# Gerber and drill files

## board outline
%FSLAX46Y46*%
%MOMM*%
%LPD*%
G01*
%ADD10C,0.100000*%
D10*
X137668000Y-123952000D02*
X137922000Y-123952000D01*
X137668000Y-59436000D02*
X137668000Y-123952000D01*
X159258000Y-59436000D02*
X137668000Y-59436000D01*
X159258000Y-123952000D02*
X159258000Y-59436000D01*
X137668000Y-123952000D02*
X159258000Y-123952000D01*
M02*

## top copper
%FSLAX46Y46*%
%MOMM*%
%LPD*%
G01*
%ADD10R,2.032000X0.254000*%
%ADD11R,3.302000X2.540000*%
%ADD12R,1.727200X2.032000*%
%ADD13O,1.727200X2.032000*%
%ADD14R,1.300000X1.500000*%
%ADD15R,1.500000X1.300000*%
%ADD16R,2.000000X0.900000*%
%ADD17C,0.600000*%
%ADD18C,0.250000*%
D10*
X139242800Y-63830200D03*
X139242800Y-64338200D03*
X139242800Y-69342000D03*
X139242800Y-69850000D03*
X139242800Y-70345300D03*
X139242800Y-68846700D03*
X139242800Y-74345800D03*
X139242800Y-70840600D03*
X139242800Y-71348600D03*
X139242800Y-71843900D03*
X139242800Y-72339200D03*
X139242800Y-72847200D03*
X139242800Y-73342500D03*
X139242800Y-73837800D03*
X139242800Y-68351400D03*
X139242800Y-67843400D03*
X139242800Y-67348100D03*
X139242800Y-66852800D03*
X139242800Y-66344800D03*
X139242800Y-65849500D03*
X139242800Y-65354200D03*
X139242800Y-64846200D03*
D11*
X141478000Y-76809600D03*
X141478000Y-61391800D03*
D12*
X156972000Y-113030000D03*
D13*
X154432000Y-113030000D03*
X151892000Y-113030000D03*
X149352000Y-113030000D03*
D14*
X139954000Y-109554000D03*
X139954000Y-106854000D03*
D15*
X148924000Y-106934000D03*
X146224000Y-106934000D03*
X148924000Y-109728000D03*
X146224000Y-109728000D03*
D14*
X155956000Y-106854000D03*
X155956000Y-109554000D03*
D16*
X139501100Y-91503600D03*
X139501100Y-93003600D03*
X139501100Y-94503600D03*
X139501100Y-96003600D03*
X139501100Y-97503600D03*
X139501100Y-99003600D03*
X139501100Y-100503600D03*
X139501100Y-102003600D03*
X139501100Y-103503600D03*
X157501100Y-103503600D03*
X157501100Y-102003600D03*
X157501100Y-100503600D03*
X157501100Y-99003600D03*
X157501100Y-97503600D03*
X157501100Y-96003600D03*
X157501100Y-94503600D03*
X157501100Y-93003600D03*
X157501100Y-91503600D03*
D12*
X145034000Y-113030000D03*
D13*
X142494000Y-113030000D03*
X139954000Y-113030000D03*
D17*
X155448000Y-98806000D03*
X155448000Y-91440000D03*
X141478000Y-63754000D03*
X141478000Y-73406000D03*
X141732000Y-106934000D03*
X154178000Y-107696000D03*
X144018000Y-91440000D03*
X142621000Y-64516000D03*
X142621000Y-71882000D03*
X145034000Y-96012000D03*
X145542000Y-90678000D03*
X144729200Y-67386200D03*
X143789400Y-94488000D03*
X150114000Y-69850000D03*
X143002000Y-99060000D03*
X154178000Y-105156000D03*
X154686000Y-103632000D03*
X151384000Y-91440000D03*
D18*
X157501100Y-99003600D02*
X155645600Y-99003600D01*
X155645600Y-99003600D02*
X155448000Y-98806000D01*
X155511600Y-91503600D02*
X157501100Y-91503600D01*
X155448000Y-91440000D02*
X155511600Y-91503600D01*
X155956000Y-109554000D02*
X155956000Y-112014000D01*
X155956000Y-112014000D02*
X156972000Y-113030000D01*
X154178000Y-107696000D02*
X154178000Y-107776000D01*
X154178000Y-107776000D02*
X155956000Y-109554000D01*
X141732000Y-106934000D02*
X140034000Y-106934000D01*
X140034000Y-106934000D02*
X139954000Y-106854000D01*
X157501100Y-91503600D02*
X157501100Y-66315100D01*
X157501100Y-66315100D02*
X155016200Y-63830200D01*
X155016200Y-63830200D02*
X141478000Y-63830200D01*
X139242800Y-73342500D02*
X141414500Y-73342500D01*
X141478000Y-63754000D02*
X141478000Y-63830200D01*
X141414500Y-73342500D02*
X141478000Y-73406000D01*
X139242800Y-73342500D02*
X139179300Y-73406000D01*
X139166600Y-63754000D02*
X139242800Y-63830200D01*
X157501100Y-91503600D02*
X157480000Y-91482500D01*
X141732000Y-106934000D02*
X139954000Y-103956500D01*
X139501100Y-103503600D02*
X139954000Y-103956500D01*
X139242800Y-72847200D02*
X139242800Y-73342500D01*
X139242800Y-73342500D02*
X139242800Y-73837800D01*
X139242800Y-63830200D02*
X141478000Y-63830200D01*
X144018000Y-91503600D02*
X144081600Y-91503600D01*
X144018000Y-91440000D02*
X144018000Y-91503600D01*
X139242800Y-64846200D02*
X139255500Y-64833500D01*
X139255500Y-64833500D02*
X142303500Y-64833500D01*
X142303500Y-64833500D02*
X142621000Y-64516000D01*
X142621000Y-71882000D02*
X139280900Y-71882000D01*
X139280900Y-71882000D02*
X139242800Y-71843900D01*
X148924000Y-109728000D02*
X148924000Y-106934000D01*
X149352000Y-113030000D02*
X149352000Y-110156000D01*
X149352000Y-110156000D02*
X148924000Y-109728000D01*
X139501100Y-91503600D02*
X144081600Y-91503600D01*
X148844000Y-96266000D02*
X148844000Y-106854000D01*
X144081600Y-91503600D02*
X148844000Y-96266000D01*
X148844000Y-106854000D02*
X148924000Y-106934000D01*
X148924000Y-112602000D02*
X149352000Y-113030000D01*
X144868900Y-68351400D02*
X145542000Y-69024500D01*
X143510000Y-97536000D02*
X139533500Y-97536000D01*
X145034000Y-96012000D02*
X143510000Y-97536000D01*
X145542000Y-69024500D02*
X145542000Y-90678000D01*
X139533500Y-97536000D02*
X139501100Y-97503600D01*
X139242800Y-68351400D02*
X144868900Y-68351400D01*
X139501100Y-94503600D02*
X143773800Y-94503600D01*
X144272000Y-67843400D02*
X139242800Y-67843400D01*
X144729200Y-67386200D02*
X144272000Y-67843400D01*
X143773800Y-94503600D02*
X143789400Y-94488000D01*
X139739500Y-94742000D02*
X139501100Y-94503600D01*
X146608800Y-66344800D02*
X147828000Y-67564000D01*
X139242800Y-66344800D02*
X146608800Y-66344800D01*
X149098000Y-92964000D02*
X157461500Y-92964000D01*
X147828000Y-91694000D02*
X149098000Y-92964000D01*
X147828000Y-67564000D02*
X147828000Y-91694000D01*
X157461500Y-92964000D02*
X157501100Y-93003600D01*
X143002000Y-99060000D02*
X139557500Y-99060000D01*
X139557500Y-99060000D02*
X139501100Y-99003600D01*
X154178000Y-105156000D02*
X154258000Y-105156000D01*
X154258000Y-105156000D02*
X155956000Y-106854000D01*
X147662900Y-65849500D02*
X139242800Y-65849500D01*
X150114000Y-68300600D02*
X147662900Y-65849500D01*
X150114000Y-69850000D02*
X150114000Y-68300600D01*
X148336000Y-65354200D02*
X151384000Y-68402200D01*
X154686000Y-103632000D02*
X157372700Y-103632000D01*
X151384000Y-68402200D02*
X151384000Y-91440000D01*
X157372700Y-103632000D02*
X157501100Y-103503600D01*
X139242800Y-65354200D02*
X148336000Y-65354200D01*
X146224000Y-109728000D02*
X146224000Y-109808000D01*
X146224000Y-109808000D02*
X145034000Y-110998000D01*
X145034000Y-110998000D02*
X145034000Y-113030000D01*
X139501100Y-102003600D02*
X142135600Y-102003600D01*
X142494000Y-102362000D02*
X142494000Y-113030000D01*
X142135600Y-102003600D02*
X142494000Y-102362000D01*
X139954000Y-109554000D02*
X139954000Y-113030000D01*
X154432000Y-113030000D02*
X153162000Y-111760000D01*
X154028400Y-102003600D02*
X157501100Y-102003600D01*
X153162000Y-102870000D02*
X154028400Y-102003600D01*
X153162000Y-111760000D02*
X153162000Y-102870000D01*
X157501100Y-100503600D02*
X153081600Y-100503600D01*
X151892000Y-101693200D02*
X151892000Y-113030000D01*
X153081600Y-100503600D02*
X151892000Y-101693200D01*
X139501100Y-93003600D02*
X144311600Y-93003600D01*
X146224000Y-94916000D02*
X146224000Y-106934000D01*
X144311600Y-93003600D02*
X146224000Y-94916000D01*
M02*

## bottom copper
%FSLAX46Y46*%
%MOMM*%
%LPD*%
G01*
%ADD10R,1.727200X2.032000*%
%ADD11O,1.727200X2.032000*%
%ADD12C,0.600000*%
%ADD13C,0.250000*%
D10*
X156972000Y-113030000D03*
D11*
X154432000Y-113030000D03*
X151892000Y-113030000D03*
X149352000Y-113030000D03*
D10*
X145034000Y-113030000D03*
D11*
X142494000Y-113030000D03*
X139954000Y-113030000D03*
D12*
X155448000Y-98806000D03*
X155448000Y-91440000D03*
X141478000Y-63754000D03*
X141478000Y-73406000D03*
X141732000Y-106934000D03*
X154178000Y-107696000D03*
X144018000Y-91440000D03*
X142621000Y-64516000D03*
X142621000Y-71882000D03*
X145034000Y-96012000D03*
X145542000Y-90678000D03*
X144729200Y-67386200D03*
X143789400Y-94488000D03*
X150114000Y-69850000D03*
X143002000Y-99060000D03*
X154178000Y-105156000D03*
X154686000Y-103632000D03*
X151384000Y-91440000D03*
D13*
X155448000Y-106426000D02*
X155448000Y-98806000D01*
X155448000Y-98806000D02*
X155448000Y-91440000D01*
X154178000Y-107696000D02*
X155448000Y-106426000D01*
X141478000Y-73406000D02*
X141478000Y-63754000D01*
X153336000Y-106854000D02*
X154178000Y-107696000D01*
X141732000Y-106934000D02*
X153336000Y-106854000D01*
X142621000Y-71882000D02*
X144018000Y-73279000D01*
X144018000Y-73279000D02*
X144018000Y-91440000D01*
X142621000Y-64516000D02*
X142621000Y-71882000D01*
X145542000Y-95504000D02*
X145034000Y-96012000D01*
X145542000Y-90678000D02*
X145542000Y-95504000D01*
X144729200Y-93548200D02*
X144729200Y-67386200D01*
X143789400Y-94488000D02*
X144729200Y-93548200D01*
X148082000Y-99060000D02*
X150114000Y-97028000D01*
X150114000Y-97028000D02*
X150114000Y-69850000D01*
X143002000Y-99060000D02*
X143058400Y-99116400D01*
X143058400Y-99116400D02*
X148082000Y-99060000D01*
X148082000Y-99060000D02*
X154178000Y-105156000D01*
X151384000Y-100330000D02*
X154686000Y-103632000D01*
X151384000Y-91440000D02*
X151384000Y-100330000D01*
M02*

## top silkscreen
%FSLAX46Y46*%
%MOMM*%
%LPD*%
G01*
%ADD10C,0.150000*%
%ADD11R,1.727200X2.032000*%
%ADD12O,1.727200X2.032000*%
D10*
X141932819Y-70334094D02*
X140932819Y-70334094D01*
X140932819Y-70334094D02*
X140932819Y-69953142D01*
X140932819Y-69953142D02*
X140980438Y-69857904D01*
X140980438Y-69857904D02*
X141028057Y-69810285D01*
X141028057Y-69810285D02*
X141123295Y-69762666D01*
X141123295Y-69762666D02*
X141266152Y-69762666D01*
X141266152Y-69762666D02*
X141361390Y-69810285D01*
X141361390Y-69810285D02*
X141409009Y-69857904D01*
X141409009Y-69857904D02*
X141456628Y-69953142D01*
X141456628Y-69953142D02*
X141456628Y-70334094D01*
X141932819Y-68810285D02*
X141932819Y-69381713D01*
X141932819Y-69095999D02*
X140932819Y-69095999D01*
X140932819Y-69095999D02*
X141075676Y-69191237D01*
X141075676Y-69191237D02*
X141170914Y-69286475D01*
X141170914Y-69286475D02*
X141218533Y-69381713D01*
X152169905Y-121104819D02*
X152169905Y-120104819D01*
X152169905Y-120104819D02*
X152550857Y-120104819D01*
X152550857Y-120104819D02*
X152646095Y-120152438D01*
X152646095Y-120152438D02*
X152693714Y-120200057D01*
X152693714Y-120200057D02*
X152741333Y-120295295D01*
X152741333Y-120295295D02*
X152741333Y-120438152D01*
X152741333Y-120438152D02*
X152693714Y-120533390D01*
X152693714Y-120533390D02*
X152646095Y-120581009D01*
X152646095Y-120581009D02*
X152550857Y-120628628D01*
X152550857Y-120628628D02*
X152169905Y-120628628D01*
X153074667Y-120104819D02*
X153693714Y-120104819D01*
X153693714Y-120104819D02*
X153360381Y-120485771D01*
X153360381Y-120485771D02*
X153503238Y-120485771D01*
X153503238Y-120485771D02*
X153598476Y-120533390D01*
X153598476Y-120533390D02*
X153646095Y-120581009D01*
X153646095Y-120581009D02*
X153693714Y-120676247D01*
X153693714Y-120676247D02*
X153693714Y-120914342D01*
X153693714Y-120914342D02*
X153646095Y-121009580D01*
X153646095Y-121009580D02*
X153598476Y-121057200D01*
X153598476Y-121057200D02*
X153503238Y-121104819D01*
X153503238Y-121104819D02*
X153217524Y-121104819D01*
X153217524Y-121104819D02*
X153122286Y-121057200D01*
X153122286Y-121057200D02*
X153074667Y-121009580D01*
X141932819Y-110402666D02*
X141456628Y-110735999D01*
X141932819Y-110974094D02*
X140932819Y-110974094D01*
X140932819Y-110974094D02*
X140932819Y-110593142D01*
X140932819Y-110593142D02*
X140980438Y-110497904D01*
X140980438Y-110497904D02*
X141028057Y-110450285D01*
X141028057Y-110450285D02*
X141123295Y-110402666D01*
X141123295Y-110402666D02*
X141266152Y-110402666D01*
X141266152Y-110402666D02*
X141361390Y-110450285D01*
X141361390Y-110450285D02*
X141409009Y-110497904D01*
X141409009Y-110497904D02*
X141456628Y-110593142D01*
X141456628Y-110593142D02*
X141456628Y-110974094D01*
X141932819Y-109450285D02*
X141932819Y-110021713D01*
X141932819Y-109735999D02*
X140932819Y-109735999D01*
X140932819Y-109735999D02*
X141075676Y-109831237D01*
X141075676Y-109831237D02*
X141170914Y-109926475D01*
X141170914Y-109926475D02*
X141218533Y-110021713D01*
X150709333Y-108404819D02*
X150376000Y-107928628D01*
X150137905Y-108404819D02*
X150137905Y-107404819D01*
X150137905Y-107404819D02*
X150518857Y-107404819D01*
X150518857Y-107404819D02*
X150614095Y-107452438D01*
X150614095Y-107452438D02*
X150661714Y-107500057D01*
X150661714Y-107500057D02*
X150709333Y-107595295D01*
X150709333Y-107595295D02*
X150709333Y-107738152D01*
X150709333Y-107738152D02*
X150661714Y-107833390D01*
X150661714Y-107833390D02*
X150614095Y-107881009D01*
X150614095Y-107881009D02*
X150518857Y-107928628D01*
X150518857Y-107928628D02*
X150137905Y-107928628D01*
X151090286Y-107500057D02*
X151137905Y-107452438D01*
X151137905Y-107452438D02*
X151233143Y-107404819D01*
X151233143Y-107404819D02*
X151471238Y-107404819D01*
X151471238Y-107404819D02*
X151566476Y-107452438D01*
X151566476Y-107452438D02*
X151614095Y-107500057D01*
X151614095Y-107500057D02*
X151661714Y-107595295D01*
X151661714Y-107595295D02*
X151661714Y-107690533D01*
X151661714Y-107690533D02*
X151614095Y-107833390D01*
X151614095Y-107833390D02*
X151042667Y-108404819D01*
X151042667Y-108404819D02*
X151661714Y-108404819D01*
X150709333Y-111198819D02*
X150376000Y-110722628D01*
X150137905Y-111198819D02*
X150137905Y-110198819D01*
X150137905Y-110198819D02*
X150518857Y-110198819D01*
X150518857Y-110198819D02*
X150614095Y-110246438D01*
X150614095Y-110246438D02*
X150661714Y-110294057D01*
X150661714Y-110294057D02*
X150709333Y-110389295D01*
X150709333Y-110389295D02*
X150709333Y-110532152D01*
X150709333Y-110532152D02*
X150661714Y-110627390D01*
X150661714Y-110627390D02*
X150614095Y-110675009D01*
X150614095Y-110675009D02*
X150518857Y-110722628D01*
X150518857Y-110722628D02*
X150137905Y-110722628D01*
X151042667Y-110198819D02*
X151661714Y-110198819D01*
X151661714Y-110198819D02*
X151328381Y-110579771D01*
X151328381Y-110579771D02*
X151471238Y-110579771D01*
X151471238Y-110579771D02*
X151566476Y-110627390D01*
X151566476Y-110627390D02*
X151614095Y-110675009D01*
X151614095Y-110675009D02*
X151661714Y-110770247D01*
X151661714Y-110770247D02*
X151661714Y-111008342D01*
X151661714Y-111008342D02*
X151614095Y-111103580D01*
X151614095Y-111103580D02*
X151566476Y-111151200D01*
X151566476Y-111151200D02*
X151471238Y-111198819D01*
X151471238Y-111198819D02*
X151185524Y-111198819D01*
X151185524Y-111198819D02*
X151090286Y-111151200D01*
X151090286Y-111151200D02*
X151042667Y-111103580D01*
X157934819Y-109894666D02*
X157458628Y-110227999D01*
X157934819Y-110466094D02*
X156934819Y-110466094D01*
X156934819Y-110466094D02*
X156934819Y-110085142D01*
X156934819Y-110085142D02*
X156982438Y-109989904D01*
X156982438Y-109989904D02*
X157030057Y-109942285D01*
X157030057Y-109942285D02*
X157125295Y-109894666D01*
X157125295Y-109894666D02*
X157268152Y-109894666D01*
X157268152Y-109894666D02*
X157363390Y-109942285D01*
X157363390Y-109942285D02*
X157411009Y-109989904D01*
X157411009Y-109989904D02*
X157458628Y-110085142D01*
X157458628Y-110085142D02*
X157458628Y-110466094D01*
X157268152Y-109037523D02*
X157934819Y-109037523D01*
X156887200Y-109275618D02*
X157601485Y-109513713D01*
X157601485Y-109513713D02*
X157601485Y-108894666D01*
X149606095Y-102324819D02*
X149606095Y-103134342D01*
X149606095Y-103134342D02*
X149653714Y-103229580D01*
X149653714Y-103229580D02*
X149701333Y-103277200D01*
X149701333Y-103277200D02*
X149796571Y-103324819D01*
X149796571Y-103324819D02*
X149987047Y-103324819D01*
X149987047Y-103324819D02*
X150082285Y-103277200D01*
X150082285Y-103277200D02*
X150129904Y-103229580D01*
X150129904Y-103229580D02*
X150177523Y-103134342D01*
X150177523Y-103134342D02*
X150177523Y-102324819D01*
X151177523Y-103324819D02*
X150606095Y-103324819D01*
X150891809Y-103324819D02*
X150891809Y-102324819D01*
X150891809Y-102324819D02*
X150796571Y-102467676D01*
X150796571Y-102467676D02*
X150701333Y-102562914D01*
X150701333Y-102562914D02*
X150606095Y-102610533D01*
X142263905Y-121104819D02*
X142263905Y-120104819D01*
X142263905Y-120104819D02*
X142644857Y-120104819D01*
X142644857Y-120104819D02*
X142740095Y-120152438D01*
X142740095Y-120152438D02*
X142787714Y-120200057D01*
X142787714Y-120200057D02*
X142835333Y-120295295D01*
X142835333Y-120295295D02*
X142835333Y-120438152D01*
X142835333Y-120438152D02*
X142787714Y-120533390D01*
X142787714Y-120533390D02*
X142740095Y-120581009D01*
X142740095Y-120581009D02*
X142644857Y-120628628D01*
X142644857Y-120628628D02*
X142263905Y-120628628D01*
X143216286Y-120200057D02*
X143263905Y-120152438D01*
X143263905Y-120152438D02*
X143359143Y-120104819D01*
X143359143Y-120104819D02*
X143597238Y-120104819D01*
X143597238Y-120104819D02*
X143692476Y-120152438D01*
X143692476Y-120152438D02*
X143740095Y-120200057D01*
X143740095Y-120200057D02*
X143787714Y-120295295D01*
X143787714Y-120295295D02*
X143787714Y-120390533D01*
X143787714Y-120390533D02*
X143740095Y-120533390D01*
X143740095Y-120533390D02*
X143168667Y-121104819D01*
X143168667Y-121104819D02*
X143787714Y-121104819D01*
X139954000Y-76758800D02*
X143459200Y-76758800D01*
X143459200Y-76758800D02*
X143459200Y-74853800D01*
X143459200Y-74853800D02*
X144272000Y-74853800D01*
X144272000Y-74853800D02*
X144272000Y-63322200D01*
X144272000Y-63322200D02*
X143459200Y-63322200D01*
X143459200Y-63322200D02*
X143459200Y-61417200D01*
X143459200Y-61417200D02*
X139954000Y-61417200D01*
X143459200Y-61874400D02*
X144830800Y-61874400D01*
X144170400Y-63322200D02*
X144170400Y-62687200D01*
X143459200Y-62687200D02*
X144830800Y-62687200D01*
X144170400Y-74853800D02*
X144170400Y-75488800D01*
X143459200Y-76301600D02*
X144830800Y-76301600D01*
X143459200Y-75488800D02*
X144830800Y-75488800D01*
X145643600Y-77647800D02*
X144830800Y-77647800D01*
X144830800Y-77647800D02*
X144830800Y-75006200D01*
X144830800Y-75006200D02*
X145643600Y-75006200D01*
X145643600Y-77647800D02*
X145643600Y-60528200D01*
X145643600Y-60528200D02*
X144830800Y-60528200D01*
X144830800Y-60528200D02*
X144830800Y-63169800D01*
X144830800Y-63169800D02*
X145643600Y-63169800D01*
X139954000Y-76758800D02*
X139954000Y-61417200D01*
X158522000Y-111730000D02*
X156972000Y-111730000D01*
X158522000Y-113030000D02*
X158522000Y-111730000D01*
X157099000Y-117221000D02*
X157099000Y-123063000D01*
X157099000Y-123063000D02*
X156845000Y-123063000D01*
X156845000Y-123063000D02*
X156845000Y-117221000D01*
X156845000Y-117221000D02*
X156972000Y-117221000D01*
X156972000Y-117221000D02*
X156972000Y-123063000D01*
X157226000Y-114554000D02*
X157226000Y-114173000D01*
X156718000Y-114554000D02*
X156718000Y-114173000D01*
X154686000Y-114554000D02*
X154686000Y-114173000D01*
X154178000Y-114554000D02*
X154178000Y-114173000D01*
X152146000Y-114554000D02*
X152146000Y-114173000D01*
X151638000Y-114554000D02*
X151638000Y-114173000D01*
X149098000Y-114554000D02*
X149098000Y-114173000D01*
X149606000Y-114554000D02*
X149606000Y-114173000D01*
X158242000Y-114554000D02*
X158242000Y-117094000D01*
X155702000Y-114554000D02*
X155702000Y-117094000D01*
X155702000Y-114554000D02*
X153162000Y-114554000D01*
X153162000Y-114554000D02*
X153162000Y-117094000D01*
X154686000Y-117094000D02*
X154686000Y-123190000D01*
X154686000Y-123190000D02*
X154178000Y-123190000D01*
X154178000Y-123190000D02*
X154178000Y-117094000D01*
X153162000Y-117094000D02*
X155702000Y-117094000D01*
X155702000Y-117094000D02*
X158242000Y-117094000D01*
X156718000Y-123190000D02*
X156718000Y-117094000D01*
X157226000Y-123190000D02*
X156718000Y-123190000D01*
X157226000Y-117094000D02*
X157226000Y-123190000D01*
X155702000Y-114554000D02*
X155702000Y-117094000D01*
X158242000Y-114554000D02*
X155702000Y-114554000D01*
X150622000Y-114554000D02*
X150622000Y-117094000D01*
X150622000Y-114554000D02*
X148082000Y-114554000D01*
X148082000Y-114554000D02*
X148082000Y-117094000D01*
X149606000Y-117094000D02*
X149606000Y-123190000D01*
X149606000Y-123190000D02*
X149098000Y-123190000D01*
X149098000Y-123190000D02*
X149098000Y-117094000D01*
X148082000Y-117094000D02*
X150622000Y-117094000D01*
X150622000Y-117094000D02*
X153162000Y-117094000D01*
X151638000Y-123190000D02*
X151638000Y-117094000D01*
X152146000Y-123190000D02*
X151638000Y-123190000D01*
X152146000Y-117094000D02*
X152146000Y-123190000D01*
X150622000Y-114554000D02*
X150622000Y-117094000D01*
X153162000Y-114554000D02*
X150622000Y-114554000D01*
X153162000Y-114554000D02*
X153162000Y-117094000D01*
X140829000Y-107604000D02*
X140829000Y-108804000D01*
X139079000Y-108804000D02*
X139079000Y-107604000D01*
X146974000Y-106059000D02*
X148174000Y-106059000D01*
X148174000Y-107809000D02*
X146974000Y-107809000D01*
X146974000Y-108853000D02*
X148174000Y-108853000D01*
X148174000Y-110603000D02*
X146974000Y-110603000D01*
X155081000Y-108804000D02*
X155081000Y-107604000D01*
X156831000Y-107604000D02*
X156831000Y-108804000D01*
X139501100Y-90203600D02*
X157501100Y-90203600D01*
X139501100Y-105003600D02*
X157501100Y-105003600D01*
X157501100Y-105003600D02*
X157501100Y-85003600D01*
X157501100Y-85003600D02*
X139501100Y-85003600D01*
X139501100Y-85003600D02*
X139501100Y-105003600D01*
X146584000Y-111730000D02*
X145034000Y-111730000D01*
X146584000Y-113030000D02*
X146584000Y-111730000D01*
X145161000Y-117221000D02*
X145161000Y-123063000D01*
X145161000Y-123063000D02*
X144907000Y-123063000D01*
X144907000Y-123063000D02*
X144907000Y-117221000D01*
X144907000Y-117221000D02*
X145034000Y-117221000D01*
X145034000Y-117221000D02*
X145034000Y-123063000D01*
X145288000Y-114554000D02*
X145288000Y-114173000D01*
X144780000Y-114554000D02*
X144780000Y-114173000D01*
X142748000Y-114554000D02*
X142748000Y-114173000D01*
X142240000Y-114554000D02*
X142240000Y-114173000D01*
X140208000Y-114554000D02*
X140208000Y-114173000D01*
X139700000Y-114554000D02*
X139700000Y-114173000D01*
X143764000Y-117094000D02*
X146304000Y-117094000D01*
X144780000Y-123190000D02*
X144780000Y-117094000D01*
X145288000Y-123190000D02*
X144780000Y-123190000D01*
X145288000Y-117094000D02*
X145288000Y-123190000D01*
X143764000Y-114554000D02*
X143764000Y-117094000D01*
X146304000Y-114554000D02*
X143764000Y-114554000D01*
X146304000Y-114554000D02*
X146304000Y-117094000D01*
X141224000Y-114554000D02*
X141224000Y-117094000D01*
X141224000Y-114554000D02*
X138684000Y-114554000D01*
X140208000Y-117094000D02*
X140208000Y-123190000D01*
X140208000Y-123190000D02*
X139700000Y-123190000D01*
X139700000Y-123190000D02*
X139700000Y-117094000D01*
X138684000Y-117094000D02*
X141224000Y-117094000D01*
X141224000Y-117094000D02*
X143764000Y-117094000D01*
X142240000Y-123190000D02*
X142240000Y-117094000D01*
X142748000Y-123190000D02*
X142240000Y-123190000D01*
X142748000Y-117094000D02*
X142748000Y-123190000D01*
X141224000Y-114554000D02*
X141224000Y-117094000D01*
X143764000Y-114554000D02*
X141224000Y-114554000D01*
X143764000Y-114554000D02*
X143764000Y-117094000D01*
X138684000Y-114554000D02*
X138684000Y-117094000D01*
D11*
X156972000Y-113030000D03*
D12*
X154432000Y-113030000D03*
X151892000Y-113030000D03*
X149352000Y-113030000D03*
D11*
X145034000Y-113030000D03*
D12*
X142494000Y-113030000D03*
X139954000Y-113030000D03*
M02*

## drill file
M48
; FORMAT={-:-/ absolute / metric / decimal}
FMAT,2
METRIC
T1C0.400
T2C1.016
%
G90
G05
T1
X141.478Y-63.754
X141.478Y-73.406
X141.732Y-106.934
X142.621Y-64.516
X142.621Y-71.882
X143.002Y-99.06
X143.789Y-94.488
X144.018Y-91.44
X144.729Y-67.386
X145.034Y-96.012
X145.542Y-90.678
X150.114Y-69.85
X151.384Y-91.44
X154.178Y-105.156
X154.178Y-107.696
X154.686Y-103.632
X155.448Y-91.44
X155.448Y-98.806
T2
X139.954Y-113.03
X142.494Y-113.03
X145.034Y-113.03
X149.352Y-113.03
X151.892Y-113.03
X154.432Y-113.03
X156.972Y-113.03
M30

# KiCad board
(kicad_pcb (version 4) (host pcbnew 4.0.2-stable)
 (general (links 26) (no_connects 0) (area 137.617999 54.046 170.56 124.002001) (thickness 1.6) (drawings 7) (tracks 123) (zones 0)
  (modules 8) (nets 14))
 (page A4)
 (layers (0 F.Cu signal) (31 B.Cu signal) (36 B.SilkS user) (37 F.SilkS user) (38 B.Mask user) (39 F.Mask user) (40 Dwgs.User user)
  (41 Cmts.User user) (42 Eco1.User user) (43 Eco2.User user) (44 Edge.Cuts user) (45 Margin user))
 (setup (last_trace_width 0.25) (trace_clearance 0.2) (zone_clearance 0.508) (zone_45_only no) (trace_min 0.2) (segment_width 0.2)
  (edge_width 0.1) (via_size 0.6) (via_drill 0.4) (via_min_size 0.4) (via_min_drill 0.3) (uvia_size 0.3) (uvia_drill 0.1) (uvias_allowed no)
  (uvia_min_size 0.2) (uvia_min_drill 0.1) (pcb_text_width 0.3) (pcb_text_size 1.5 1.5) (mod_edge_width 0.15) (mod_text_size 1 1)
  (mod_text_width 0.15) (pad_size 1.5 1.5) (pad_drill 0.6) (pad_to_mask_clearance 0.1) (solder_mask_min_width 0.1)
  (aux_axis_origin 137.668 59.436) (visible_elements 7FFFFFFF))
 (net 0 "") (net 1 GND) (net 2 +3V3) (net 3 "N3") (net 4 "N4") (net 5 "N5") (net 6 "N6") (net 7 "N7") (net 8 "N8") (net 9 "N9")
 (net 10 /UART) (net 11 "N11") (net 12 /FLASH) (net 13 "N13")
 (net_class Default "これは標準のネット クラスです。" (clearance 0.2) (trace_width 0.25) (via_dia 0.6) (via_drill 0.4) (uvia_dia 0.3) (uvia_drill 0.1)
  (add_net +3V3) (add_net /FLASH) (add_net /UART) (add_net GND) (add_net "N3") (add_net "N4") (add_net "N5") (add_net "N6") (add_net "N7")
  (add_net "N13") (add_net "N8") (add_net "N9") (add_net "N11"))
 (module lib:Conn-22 (layer F.Cu) (at 142.494 69.088 90)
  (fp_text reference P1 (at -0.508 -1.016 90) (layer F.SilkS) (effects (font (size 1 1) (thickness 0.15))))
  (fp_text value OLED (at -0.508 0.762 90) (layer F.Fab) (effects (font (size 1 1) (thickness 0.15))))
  (fp_line (start -7.6708 -2.54) (end -7.6708 0.9652) (layer F.SilkS) (width 0.15))
  (fp_line (start -7.6708 0.9652) (end -5.7658 0.9652) (layer F.SilkS) (width 0.15))
  (fp_line (start -5.7658 0.9652) (end -5.7658 1.778) (layer F.SilkS) (width 0.15))
  (fp_line (start -5.7658 1.778) (end 5.7658 1.778) (layer F.SilkS) (width 0.15))
  (fp_line (start 5.7658 1.778) (end 5.7658 0.9652) (layer F.SilkS) (width 0.15))
  (fp_line (start 5.7658 0.9652) (end 7.6708 0.9652) (layer F.SilkS) (width 0.15))
  (fp_line (start 7.6708 0.9652) (end 7.6708 -2.54) (layer F.SilkS) (width 0.15))
  (fp_line (start 7.2136 0.9652) (end 7.2136 2.3368) (layer F.SilkS) (width 0.15))
  (fp_line (start 5.7658 1.6764) (end 6.4008 1.6764) (layer F.SilkS) (width 0.15))
  (fp_line (start 6.4008 0.9652) (end 6.4008 2.3368) (layer F.SilkS) (width 0.15))
  (fp_line (start -5.7658 1.6764) (end -6.4008 1.6764) (layer F.SilkS) (width 0.15))
  (fp_line (start -7.2136 0.9652) (end -7.2136 2.3368) (layer F.SilkS) (width 0.15))
  (fp_line (start -6.4008 0.9652) (end -6.4008 2.3368) (layer F.SilkS) (width 0.15))
  (fp_line (start -8.5598 3.1496) (end -8.5598 2.3368) (layer F.SilkS) (width 0.15))
  (fp_line (start -8.5598 2.3368) (end -5.9182 2.3368) (layer F.SilkS) (width 0.15))
  (fp_line (start -5.9182 2.3368) (end -5.9182 3.1496) (layer F.SilkS) (width 0.15))
  (fp_line (start -8.5598 3.1496) (end 8.5598 3.1496) (layer F.SilkS) (width 0.15))
  (fp_line (start 8.5598 3.1496) (end 8.5598 2.3368) (layer F.SilkS) (width 0.15))
  (fp_line (start 8.5598 2.3368) (end 5.9182 2.3368) (layer F.SilkS) (width 0.15))
  (fp_line (start 5.9182 2.3368) (end 5.9182 3.1496) (layer F.SilkS) (width 0.15))
  (fp_line (start -7.6708 -2.54) (end 7.6708 -2.54) (layer F.SilkS) (width 0.15))
  (pad 22 smd rect (at 5.2578 -3.2512 90) (size 0.254 2.032) (layers F.Cu F.Mask) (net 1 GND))
  (pad 21 smd rect (at 4.7498 -3.2512 90) (size 0.254 2.032) (layers F.Cu F.Mask))
  (pad 11 smd rect (at -0.254 -3.2512 90) (size 0.254 2.032) (layers F.Cu F.Mask))
  (pad 10 smd rect (at -0.762 -3.2512 90) (size 0.254 2.032) (layers F.Cu F.Mask))
  (pad 9 smd rect (at -1.2573 -3.2512 90) (size 0.254 2.032) (layers F.Cu F.Mask))
  (pad 12 smd rect (at 0.2413 -3.2512 90) (size 0.254 2.032) (layers F.Cu F.Mask))
  (pad 1 smd rect (at -5.2578 -3.2512 90) (size 0.254 2.032) (layers F.Cu F.Mask))
  (pad 8 smd rect (at -1.7526 -3.2512 90) (size 0.254 2.032) (layers F.Cu F.Mask))
  (pad 7 smd rect (at -2.2606 -3.2512 90) (size 0.254 2.032) (layers F.Cu F.Mask))
  (pad 6 smd rect (at -2.7559 -3.2512 90) (size 0.254 2.032) (layers F.Cu F.Mask) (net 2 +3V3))
  (pad 5 smd rect (at -3.2512 -3.2512 90) (size 0.254 2.032) (layers F.Cu F.Mask))
  (pad 4 smd rect (at -3.7592 -3.2512 90) (size 0.254 2.032) (layers F.Cu F.Mask) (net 1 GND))
  (pad 3 smd rect (at -4.2545 -3.2512 90) (size 0.254 2.032) (layers F.Cu F.Mask) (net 1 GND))
  (pad 2 smd rect (at -4.7498 -3.2512 90) (size 0.254 2.032) (layers F.Cu F.Mask) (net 1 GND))
  (pad 13 smd rect (at 0.7366 -3.2512 90) (size 0.254 2.032) (layers F.Cu F.Mask) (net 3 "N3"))
  (pad 14 smd rect (at 1.2446 -3.2512 90) (size 0.254 2.032) (layers F.Cu F.Mask) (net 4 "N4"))
  (pad 15 smd rect (at 1.7399 -3.2512 90) (size 0.254 2.032) (layers F.Cu F.Mask))
  (pad 16 smd rect (at 2.2352 -3.2512 90) (size 0.254 2.032) (layers F.Cu F.Mask))
  (pad 17 smd rect (at 2.7432 -3.2512 90) (size 0.254 2.032) (layers F.Cu F.Mask) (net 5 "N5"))
  (pad 18 smd rect (at 3.2385 -3.2512 90) (size 0.254 2.032) (layers F.Cu F.Mask) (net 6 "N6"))
  (pad 19 smd rect (at 3.7338 -3.2512 90) (size 0.254 2.032) (layers F.Cu F.Mask) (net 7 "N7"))
  (pad 20 smd rect (at 4.2418 -3.2512 90) (size 0.254 2.032) (layers F.Cu F.Mask) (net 2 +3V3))
  (pad "" smd rect (at -7.7216 -1.016 90) (size 2.54 3.302) (layers F.Cu F.Mask))
  (pad "" smd rect (at 7.6962 -1.016 90) (size 2.54 3.302) (layers F.Cu F.Mask)))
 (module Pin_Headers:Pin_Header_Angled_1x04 (layer F.Cu) (at 156.972 113.03 270)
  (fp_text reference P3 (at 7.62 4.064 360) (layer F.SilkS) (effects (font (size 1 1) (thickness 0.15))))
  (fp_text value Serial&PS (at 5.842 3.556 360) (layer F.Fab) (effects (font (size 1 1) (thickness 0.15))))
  (fp_line (start -1.3 -1.55) (end -1.3 0) (layer F.SilkS) (width 0.15))
  (fp_line (start 0 -1.55) (end -1.3 -1.55) (layer F.SilkS) (width 0.15))
  (fp_line (start 4.191 -0.127) (end 10.033 -0.127) (layer F.SilkS) (width 0.15))
  (fp_line (start 10.033 -0.127) (end 10.033 0.127) (layer F.SilkS) (width 0.15))
  (fp_line (start 10.033 0.127) (end 4.191 0.127) (layer F.SilkS) (width 0.15))
  (fp_line (start 4.191 0.127) (end 4.191 0) (layer F.SilkS) (width 0.15))
  (fp_line (start 4.191 0) (end 10.033 0) (layer F.SilkS) (width 0.15))
  (fp_line (start 1.524 -0.254) (end 1.143 -0.254) (layer F.SilkS) (width 0.15))
  (fp_line (start 1.524 0.254) (end 1.143 0.254) (layer F.SilkS) (width 0.15))
  (fp_line (start 1.524 2.286) (end 1.143 2.286) (layer F.SilkS) (width 0.15))
  (fp_line (start 1.524 2.794) (end 1.143 2.794) (layer F.SilkS) (width 0.15))
  (fp_line (start 1.524 4.826) (end 1.143 4.826) (layer F.SilkS) (width 0.15))
  (fp_line (start 1.524 5.334) (end 1.143 5.334) (layer F.SilkS) (width 0.15))
  (fp_line (start 1.524 7.874) (end 1.143 7.874) (layer F.SilkS) (width 0.15))
  (fp_line (start 1.524 7.366) (end 1.143 7.366) (layer F.SilkS) (width 0.15))
  (fp_line (start 1.524 -1.27) (end 4.064 -1.27) (layer F.SilkS) (width 0.15))
  (fp_line (start 1.524 1.27) (end 4.064 1.27) (layer F.SilkS) (width 0.15))
  (fp_line (start 1.524 1.27) (end 1.524 3.81) (layer F.SilkS) (width 0.15))
  (fp_line (start 1.524 3.81) (end 4.064 3.81) (layer F.SilkS) (width 0.15))
  (fp_line (start 4.064 2.286) (end 10.16 2.286) (layer F.SilkS) (width 0.15))
  (fp_line (start 10.16 2.286) (end 10.16 2.794) (layer F.SilkS) (width 0.15))
  (fp_line (start 10.16 2.794) (end 4.064 2.794) (layer F.SilkS) (width 0.15))
  (fp_line (start 4.064 3.81) (end 4.064 1.27) (layer F.SilkS) (width 0.15))
  (fp_line (start 4.064 1.27) (end 4.064 -1.27) (layer F.SilkS) (width 0.15))
  (fp_line (start 10.16 0.254) (end 4.064 0.254) (layer F.SilkS) (width 0.15))
  (fp_line (start 10.16 -0.254) (end 10.16 0.254) (layer F.SilkS) (width 0.15))
  (fp_line (start 4.064 -0.254) (end 10.16 -0.254) (layer F.SilkS) (width 0.15))
  (fp_line (start 1.524 1.27) (end 4.064 1.27) (layer F.SilkS) (width 0.15))
  (fp_line (start 1.524 -1.27) (end 1.524 1.27) (layer F.SilkS) (width 0.15))
  (fp_line (start 1.524 6.35) (end 4.064 6.35) (layer F.SilkS) (width 0.15))
  (fp_line (start 1.524 6.35) (end 1.524 8.89) (layer F.SilkS) (width 0.15))
  (fp_line (start 1.524 8.89) (end 4.064 8.89) (layer F.SilkS) (width 0.15))
  (fp_line (start 4.064 7.366) (end 10.16 7.366) (layer F.SilkS) (width 0.15))
  (fp_line (start 10.16 7.366) (end 10.16 7.874) (layer F.SilkS) (width 0.15))
  (fp_line (start 10.16 7.874) (end 4.064 7.874) (layer F.SilkS) (width 0.15))
  (fp_line (start 4.064 8.89) (end 4.064 6.35) (layer F.SilkS) (width 0.15))
  (fp_line (start 4.064 6.35) (end 4.064 3.81) (layer F.SilkS) (width 0.15))
  (fp_line (start 10.16 5.334) (end 4.064 5.334) (layer F.SilkS) (width 0.15))
  (fp_line (start 10.16 4.826) (end 10.16 5.334) (layer F.SilkS) (width 0.15))
  (fp_line (start 4.064 4.826) (end 10.16 4.826) (layer F.SilkS) (width 0.15))
  (fp_line (start 1.524 6.35) (end 4.064 6.35) (layer F.SilkS) (width 0.15))
  (fp_line (start 1.524 3.81) (end 1.524 6.35) (layer F.SilkS) (width 0.15))
  (fp_line (start 1.524 3.81) (end 4.064 3.81) (layer F.SilkS) (width 0.15))
  (pad 1 thru_hole rect (at 0 0 270) (size 2.032 1.7272) (drill 1.016) (layers *.Cu *.Mask F.SilkS) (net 1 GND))
  (pad 2 thru_hole oval (at 0 2.54 270) (size 2.032 1.7272) (drill 1.016) (layers *.Cu *.Mask F.SilkS) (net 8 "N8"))
  (pad 3 thru_hole oval (at 0 5.08 270) (size 2.032 1.7272) (drill 1.016) (layers *.Cu *.Mask F.SilkS) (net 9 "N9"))
  (pad 4 thru_hole oval (at 0 7.62 270) (size 2.032 1.7272) (drill 1.016) (layers *.Cu *.Mask F.SilkS) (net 2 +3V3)))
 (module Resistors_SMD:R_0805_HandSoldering (layer F.Cu) (at 139.954 108.204 90)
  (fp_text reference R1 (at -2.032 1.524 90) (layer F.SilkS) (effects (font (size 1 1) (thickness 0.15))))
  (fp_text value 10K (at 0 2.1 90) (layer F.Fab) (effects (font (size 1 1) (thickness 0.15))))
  (fp_line (start 0.6 0.875) (end -0.6 0.875) (layer F.SilkS) (width 0.15))
  (fp_line (start -0.6 -0.875) (end 0.6 -0.875) (layer F.SilkS) (width 0.15))
  (pad 1 smd rect (at -1.35 0 90) (size 1.5 1.3) (layers F.Cu F.Mask) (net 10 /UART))
  (pad 2 smd rect (at 1.35 0 90) (size 1.5 1.3) (layers F.Cu F.Mask) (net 1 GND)))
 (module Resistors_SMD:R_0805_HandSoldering (layer F.Cu) (at 147.574 106.934 180)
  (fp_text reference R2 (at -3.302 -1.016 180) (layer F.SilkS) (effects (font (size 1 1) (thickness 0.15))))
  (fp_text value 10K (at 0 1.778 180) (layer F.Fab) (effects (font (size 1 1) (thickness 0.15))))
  (fp_line (start 0.6 0.875) (end -0.6 0.875) (layer F.SilkS) (width 0.15))
  (fp_line (start -0.6 -0.875) (end 0.6 -0.875) (layer F.SilkS) (width 0.15))
  (pad 1 smd rect (at -1.35 0 180) (size 1.5 1.3) (layers F.Cu F.Mask) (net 2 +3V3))
  (pad 2 smd rect (at 1.35 0 180) (size 1.5 1.3) (layers F.Cu F.Mask) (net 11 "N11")))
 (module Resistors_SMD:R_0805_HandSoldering (layer F.Cu) (at 147.574 109.728 180)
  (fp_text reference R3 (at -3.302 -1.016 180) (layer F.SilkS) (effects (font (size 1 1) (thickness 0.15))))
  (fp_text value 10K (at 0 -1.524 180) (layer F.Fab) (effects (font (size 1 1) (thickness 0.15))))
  (fp_line (start 0.6 0.875) (end -0.6 0.875) (layer F.SilkS) (width 0.15))
  (fp_line (start -0.6 -0.875) (end 0.6 -0.875) (layer F.SilkS) (width 0.15))
  (pad 1 smd rect (at -1.35 0 180) (size 1.5 1.3) (layers F.Cu F.Mask) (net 2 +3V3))
  (pad 2 smd rect (at 1.35 0 180) (size 1.5 1.3) (layers F.Cu F.Mask) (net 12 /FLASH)))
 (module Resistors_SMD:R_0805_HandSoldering (layer F.Cu) (at 155.956 108.204 270)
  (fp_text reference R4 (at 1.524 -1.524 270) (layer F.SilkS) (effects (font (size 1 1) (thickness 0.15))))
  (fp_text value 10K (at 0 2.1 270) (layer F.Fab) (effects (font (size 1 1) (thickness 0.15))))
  (fp_line (start 0.6 0.875) (end -0.6 0.875) (layer F.SilkS) (width 0.15))
  (fp_line (start -0.6 -0.875) (end 0.6 -0.875) (layer F.SilkS) (width 0.15))
  (pad 1 smd rect (at -1.35 0 270) (size 1.5 1.3) (layers F.Cu F.Mask) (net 6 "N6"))
  (pad 2 smd rect (at 1.35 0 270) (size 1.5 1.3) (layers F.Cu F.Mask) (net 1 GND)))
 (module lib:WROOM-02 (layer F.Cu) (at 148.5011 105.0036)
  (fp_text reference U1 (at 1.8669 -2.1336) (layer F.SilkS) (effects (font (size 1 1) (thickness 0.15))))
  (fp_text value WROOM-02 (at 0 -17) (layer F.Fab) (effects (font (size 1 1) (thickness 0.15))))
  (fp_line (start -9 -14.8) (end 9 -14.8) (layer F.SilkS) (width 0.15))
  (fp_line (start -9 0) (end 9 0) (layer F.SilkS) (width 0.15))
  (fp_line (start 9 0) (end 9 -20) (layer F.SilkS) (width 0.15))
  (fp_line (start 9 -20) (end -9 -20) (layer F.SilkS) (width 0.15))
  (fp_line (start -9 -20) (end -9 0) (layer F.SilkS) (width 0.15))
  (pad 1 smd rect (at -9 -13.5) (size 2 0.9) (layers F.Cu F.Mask) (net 2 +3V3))
  (pad 2 smd rect (at -9 -12) (size 2 0.9) (layers F.Cu F.Mask) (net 11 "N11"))
  (pad 3 smd rect (at -9 -10.5) (size 2 0.9) (layers F.Cu F.Mask) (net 4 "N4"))
  (pad 4 smd rect (at -9 -9) (size 2 0.9) (layers F.Cu F.Mask))
  (pad 5 smd rect (at -9 -7.5) (size 2 0.9) (layers F.Cu F.Mask) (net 3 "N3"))
  (pad 6 smd rect (at -9 -6) (size 2 0.9) (layers F.Cu F.Mask) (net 6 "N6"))
  (pad 7 smd rect (at -9 -4.5) (size 2 0.9) (layers F.Cu F.Mask))
  (pad 8 smd rect (at -9 -3) (size 2 0.9) (layers F.Cu F.Mask) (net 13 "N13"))
  (pad 9 smd rect (at -9 -1.5) (size 2 0.9) (layers F.Cu F.Mask) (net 1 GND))
  (pad 10 smd rect (at 9 -1.5) (size 2 0.9) (layers F.Cu F.Mask) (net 7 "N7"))
  (pad 11 smd rect (at 9 -3) (size 2 0.9) (layers F.Cu F.Mask) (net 8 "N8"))
  (pad 12 smd rect (at 9 -4.5) (size 2 0.9) (layers F.Cu F.Mask) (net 9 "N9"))
  (pad 13 smd rect (at 9 -6) (size 2 0.9) (layers F.Cu F.Mask) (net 1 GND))
  (pad 14 smd rect (at 9 -7.5) (size 2 0.9) (layers F.Cu F.Mask))
  (pad 15 smd rect (at 9 -9) (size 2 0.9) (layers F.Cu F.Mask))
  (pad 16 smd rect (at 9 -10.5) (size 2 0.9) (layers F.Cu F.Mask))
  (pad 17 smd rect (at 9 -12) (size 2 0.9) (layers F.Cu F.Mask) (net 5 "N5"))
  (pad 18 smd rect (at 9 -13.5) (size 2 0.9) (layers F.Cu F.Mask) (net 1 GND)))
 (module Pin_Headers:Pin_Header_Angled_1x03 (layer F.Cu) (at 145.034 113.03 270)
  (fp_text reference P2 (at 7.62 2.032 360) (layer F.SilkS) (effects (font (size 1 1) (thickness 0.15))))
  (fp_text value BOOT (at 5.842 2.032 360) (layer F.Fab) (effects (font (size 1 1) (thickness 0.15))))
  (fp_line (start -1.3 -1.55) (end -1.3 0) (layer F.SilkS) (width 0.15))
  (fp_line (start 0 -1.55) (end -1.3 -1.55) (layer F.SilkS) (width 0.15))
  (fp_line (start 4.191 -0.127) (end 10.033 -0.127) (layer F.SilkS) (width 0.15))
  (fp_line (start 10.033 -0.127) (end 10.033 0.127) (layer F.SilkS) (width 0.15))
  (fp_line (start 10.033 0.127) (end 4.191 0.127) (layer F.SilkS) (width 0.15))
  (fp_line (start 4.191 0.127) (end 4.191 0) (layer F.SilkS) (width 0.15))
  (fp_line (start 4.191 0) (end 10.033 0) (layer F.SilkS) (width 0.15))
  (fp_line (start 1.524 -0.254) (end 1.143 -0.254) (layer F.SilkS) (width 0.15))
  (fp_line (start 1.524 0.254) (end 1.143 0.254) (layer F.SilkS) (width 0.15))
  (fp_line (start 1.524 2.286) (end 1.143 2.286) (layer F.SilkS) (width 0.15))
  (fp_line (start 1.524 2.794) (end 1.143 2.794) (layer F.SilkS) (width 0.15))
  (fp_line (start 1.524 4.826) (end 1.143 4.826) (layer F.SilkS) (width 0.15))
  (fp_line (start 1.524 5.334) (end 1.143 5.334) (layer F.SilkS) (width 0.15))
  (fp_line (start 4.064 1.27) (end 4.064 -1.27) (layer F.SilkS) (width 0.15))
  (fp_line (start 10.16 0.254) (end 4.064 0.254) (layer F.SilkS) (width 0.15))
  (fp_line (start 10.16 -0.254) (end 10.16 0.254) (layer F.SilkS) (width 0.15))
  (fp_line (start 4.064 -0.254) (end 10.16 -0.254) (layer F.SilkS) (width 0.15))
  (fp_line (start 1.524 1.27) (end 4.064 1.27) (layer F.SilkS) (width 0.15))
  (fp_line (start 1.524 -1.27) (end 1.524 1.27) (layer F.SilkS) (width 0.15))
  (fp_line (start 1.524 -1.27) (end 4.064 -1.27) (layer F.SilkS) (width 0.15))
  (fp_line (start 1.524 3.81) (end 4.064 3.81) (layer F.SilkS) (width 0.15))
  (fp_line (start 1.524 3.81) (end 1.524 6.35) (layer F.SilkS) (width 0.15))
  (fp_line (start 4.064 4.826) (end 10.16 4.826) (layer F.SilkS) (width 0.15))
  (fp_line (start 10.16 4.826) (end 10.16 5.334) (layer F.SilkS) (width 0.15))
  (fp_line (start 10.16 5.334) (end 4.064 5.334) (layer F.SilkS) (width 0.15))
  (fp_line (start 4.064 6.35) (end 4.064 3.81) (layer F.SilkS) (width 0.15))
  (fp_line (start 4.064 3.81) (end 4.064 1.27) (layer F.SilkS) (width 0.15))
  (fp_line (start 10.16 2.794) (end 4.064 2.794) (layer F.SilkS) (width 0.15))
  (fp_line (start 10.16 2.286) (end 10.16 2.794) (layer F.SilkS) (width 0.15))
  (fp_line (start 4.064 2.286) (end 10.16 2.286) (layer F.SilkS) (width 0.15))
  (fp_line (start 1.524 3.81) (end 4.064 3.81) (layer F.SilkS) (width 0.15))
  (fp_line (start 1.524 1.27) (end 1.524 3.81) (layer F.SilkS) (width 0.15))
  (fp_line (start 1.524 1.27) (end 4.064 1.27) (layer F.SilkS) (width 0.15))
  (fp_line (start 1.524 6.35) (end 4.064 6.35) (layer F.SilkS) (width 0.15))
  (pad 1 thru_hole rect (at 0 0 270) (size 2.032 1.7272) (drill 1.016) (layers *.Cu *.Mask F.SilkS) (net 12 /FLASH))
  (pad 2 thru_hole oval (at 0 2.54 270) (size 2.032 1.7272) (drill 1.016) (layers *.Cu *.Mask F.SilkS) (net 13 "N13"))
  (pad 3 thru_hole oval (at 0 5.08 270) (size 2.032 1.7272) (drill 1.016) (layers *.Cu *.Mask F.SilkS) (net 10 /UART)))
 (gr_line (start 137.668 123.952) (end 137.922 123.952) (angle 90) (layer Edge.Cuts) (width 0.1))
 (gr_line (start 137.668 59.436) (end 137.668 123.952) (angle 90) (layer Edge.Cuts) (width 0.1))
 (gr_line (start 159.258 59.436) (end 137.668 59.436) (angle 90) (layer Edge.Cuts) (width 0.1))
 (gr_line (start 159.258 123.952) (end 159.258 59.436) (angle 90) (layer Edge.Cuts) (width 0.1))
 (gr_line (start 137.668 123.952) (end 159.258 123.952) (angle 90) (layer Edge.Cuts) (width 0.1))
 (segment (start 157.5011 99.0036) (end 155.6456 99.0036) (width 0.25) (layer F.Cu) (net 1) (status 10))
 (via (at 155.448 98.806) (size 0.6) (drill 0.4) (layers F.Cu B.Cu) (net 1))
 (segment (start 155.6456 99.0036) (end 155.448 98.806) (width 0.25) (layer F.Cu) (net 1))
 (via (at 155.448 91.44) (size 0.6) (drill 0.4) (layers F.Cu B.Cu) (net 1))
 (segment (start 155.448 106.426) (end 155.448 98.806) (width 0.25) (layer B.Cu) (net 1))
 (segment (start 155.448 98.806) (end 155.448 91.44) (width 0.25) (layer B.Cu) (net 1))
 (segment (start 154.178 107.696) (end 155.448 106.426) (width 0.25) (layer B.Cu) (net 1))
 (segment (start 155.5116 91.5036) (end 157.5011 91.5036) (width 0.25) (layer F.Cu) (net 1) (status 20))
 (segment (start 155.448 91.44) (end 155.5116 91.5036) (width 0.25) (layer F.Cu) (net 1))
 (segment (start 155.956 109.554) (end 155.956 112.014) (width 0.25) (layer F.Cu) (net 1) (status 10))
 (segment (start 155.956 112.014) (end 156.972 113.03) (width 0.25) (layer F.Cu) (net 1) (status 20))
 (segment (start 154.178 107.696) (end 154.178 107.776) (width 0.25) (layer F.Cu) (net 1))
 (segment (start 154.178 107.776) (end 155.956 109.554) (width 0.25) (layer F.Cu) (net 1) (status 20))
 (segment (start 141.732 106.934) (end 140.034 106.934) (width 0.25) (layer F.Cu) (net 1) (status 20))
 (segment (start 140.034 106.934) (end 139.954 106.854) (width 0.25) (layer F.Cu) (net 1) (status 30))
 (segment (start 157.5011 91.5036) (end 157.5011 66.3151) (width 0.25) (layer F.Cu) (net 1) (status 10))
 (segment (start 157.5011 66.3151) (end 155.0162 63.8302) (width 0.25) (layer F.Cu) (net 1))
 (segment (start 155.0162 63.8302) (end 141.478 63.8302) (width 0.25) (layer F.Cu) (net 1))
 (segment (start 139.2428 73.3425) (end 141.4145 73.3425) (width 0.25) (layer F.Cu) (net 1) (status 10))
 (segment (start 141.478 63.754) (end 141.478 63.8302) (width 0.25) (layer F.Cu) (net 1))
 (via (at 141.478 63.754) (size 0.6) (drill 0.4) (layers F.Cu B.Cu) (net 1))
 (segment (start 141.478 73.406) (end 141.478 63.754) (width 0.25) (layer B.Cu) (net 1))
 (via (at 141.478 73.406) (size 0.6) (drill 0.4) (layers F.Cu B.Cu) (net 1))
 (segment (start 141.4145 73.3425) (end 141.478 73.406) (width 0.25) (layer F.Cu) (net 1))
 (segment (start 139.2428 73.3425) (end 139.1793 73.406) (width 0.25) (layer F.Cu) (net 1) (status 30))
 (segment (start 139.1666 63.754) (end 139.2428 63.8302) (width 0.25) (layer F.Cu) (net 1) (status 30))
 (segment (start 157.5011 91.5036) (end 157.48 91.4825) (width 0.25) (layer F.Cu) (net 1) (status 30))
 (via (at 141.732 106.934) (size 0.6) (drill 0.4) (layers F.Cu B.Cu) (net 1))
 (segment (start 141.732 106.934) (end 139.954 103.9565) (width 0.25) (layer F.Cu) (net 1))
 (segment (start 139.5011 103.5036) (end 139.954 103.9565) (width 0.25) (layer F.Cu) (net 1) (status 10))
 (via (at 154.178 107.696) (size 0.6) (drill 0.4) (layers F.Cu B.Cu) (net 1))
 (segment (start 153.336 106.854) (end 154.178 107.696) (width 0.25) (layer B.Cu) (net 1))
 (segment (start 141.732 106.934) (end 153.336 106.854) (width 0.25) (layer B.Cu) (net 1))
 (segment (start 139.2428 72.8472) (end 139.2428 73.3425) (width 0.25) (layer F.Cu) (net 1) (status 30))
 (segment (start 139.2428 73.3425) (end 139.2428 73.8378) (width 0.25) (layer F.Cu) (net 1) (status 30))
 (segment (start 139.2428 63.8302) (end 141.478 63.8302) (width 0.25) (layer F.Cu) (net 1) (status 10))
 (segment (start 142.621 71.882) (end 144.018 73.279) (width 0.25) (layer B.Cu) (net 2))
 (segment (start 144.018 91.5036) (end 144.0816 91.5036) (width 0.25) (layer F.Cu) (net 2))
 (segment (start 144.018 91.44) (end 144.018 91.5036) (width 0.25) (layer F.Cu) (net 2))
 (via (at 144.018 91.44) (size 0.6) (drill 0.4) (layers F.Cu B.Cu) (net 2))
 (segment (start 144.018 73.279) (end 144.018 91.44) (width 0.25) (layer B.Cu) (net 2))
 (segment (start 139.2428 64.8462) (end 139.2555 64.8335) (width 0.25) (layer F.Cu) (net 2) (status 30))
 (segment (start 139.2555 64.8335) (end 142.3035 64.8335) (width 0.25) (layer F.Cu) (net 2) (status 10))
 (segment (start 142.3035 64.8335) (end 142.621 64.516) (width 0.25) (layer F.Cu) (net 2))
 (via (at 142.621 64.516) (size 0.6) (drill 0.4) (layers F.Cu B.Cu) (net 2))
 (segment (start 142.621 64.516) (end 142.621 71.882) (width 0.25) (layer B.Cu) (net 2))
 (via (at 142.621 71.882) (size 0.6) (drill 0.4) (layers F.Cu B.Cu) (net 2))
 (segment (start 142.621 71.882) (end 139.2809 71.882) (width 0.25) (layer F.Cu) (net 2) (status 20))
 (segment (start 139.2809 71.882) (end 139.2428 71.8439) (width 0.25) (layer F.Cu) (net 2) (status 30))
 (segment (start 148.924 109.728) (end 148.924 106.934) (width 0.25) (layer F.Cu) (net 2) (status 30))
 (segment (start 149.352 113.03) (end 149.352 110.156) (width 0.25) (layer F.Cu) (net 2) (status 30))
 (segment (start 149.352 110.156) (end 148.924 109.728) (width 0.25) (layer F.Cu) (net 2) (status 30))
 (segment (start 139.5011 91.5036) (end 144.0816 91.5036) (width 0.25) (layer F.Cu) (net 2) (status 10))
 (segment (start 148.844 96.266) (end 148.844 106.854) (width 0.25) (layer F.Cu) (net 2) (status 20))
 (segment (start 144.0816 91.5036) (end 148.844 96.266) (width 0.25) (layer F.Cu) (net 2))
 (segment (start 148.844 106.854) (end 148.924 106.934) (width 0.25) (layer F.Cu) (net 2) (status 30))
 (segment (start 148.924 112.602) (end 149.352 113.03) (width 0.25) (layer F.Cu) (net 2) (status 30))
 (segment (start 144.8689 68.3514) (end 145.542 69.0245) (width 0.25) (layer F.Cu) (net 3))
 (segment (start 143.51 97.536) (end 139.5335 97.536) (width 0.25) (layer F.Cu) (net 3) (status 20))
 (segment (start 145.034 96.012) (end 143.51 97.536) (width 0.25) (layer F.Cu) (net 3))
 (via (at 145.034 96.012) (size 0.6) (drill 0.4) (layers F.Cu B.Cu) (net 3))
 (segment (start 145.542 95.504) (end 145.034 96.012) (width 0.25) (layer B.Cu) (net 3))
 (segment (start 145.542 90.678) (end 145.542 95.504) (width 0.25) (layer B.Cu) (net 3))
 (via (at 145.542 90.678) (size 0.6) (drill 0.4) (layers F.Cu B.Cu) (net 3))
 (segment (start 145.542 69.0245) (end 145.542 90.678) (width 0.25) (layer F.Cu) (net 3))
 (segment (start 139.5335 97.536) (end 139.5011 97.5036) (width 0.25) (layer F.Cu) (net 3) (status 30))
 (segment (start 139.2428 68.3514) (end 144.8689 68.3514) (width 0.25) (layer F.Cu) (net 3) (status 10))
 (segment (start 139.5011 94.5036) (end 143.7738 94.5036) (width 0.25) (layer F.Cu) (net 4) (status 10))
 (segment (start 144.272 67.8434) (end 139.2428 67.8434) (width 0.25) (layer F.Cu) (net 4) (status 20))
 (segment (start 144.7292 67.3862) (end 144.272 67.8434) (width 0.25) (layer F.Cu) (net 4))
 (via (at 144.7292 67.3862) (size 0.6) (drill 0.4) (layers F.Cu B.Cu) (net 4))
 (segment (start 144.7292 93.5482) (end 144.7292 67.3862) (width 0.25) (layer B.Cu) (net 4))
 (segment (start 143.7894 94.488) (end 144.7292 93.5482) (width 0.25) (layer B.Cu) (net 4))
 (via (at 143.7894 94.488) (size 0.6) (drill 0.4) (layers F.Cu B.Cu) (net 4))
 (segment (start 143.7738 94.5036) (end 143.7894 94.488) (width 0.25) (layer F.Cu) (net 4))
 (segment (start 139.7395 94.742) (end 139.5011 94.5036) (width 0.25) (layer F.Cu) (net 4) (status 30))
 (segment (start 146.6088 66.3448) (end 147.828 67.564) (width 0.25) (layer F.Cu) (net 5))
 (segment (start 139.2428 66.3448) (end 146.6088 66.3448) (width 0.25) (layer F.Cu) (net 5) (status 10))
 (segment (start 149.098 92.964) (end 157.4615 92.964) (width 0.25) (layer F.Cu) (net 5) (status 20))
 (segment (start 147.828 91.694) (end 149.098 92.964) (width 0.25) (layer F.Cu) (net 5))
 (segment (start 147.828 67.564) (end 147.828 91.694) (width 0.25) (layer F.Cu) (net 5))
 (segment (start 157.4615 92.964) (end 157.5011 93.0036) (width 0.25) (layer F.Cu) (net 5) (status 30))
 (segment (start 143.002 99.06) (end 139.5575 99.06) (width 0.25) (layer F.Cu) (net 6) (status 20))
 (segment (start 139.5575 99.06) (end 139.5011 99.0036) (width 0.25) (layer F.Cu) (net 6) (status 30))
 (segment (start 154.178 105.156) (end 154.258 105.156) (width 0.25) (layer F.Cu) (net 6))
 (segment (start 154.258 105.156) (end 155.956 106.854) (width 0.25) (layer F.Cu) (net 6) (status 20))
 (segment (start 148.082 99.06) (end 150.114 97.028) (width 0.25) (layer B.Cu) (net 6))
 (segment (start 147.6629 65.8495) (end 139.2428 65.8495) (width 0.25) (layer F.Cu) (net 6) (status 20))
 (segment (start 150.114 68.3006) (end 147.6629 65.8495) (width 0.25) (layer F.Cu) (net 6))
 (segment (start 150.114 69.85) (end 150.114 68.3006) (width 0.25) (layer F.Cu) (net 6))
 (via (at 150.114 69.85) (size 0.6) (drill 0.4) (layers F.Cu B.Cu) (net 6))
 (segment (start 150.114 97.028) (end 150.114 69.85) (width 0.25) (layer B.Cu) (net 6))
 (via (at 143.002 99.06) (size 0.6) (drill 0.4) (layers F.Cu B.Cu) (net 6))
 (segment (start 143.002 99.06) (end 143.0584 99.1164) (width 0.25) (layer B.Cu) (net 6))
 (segment (start 143.0584 99.1164) (end 148.082 99.06) (width 0.25) (layer B.Cu) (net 6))
 (via (at 154.178 105.156) (size 0.6) (drill 0.4) (layers F.Cu B.Cu) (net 6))
 (segment (start 148.082 99.06) (end 154.178 105.156) (width 0.25) (layer B.Cu) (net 6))
 (segment (start 148.336 65.3542) (end 151.384 68.4022) (width 0.25) (layer F.Cu) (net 7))
 (segment (start 154.686 103.632) (end 157.3727 103.632) (width 0.25) (layer F.Cu) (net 7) (status 20))
 (via (at 154.686 103.632) (size 0.6) (drill 0.4) (layers F.Cu B.Cu) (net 7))
 (segment (start 151.384 100.33) (end 154.686 103.632) (width 0.25) (layer B.Cu) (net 7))
 (segment (start 151.384 91.44) (end 151.384 100.33) (width 0.25) (layer B.Cu) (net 7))
 (via (at 151.384 91.44) (size 0.6) (drill 0.4) (layers F.Cu B.Cu) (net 7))
 (segment (start 151.384 68.4022) (end 151.384 91.44) (width 0.25) (layer F.Cu) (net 7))
 (segment (start 157.3727 103.632) (end 157.5011 103.5036) (width 0.25) (layer F.Cu) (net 7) (status 30))
 (segment (start 139.2428 65.3542) (end 148.336 65.3542) (width 0.25) (layer F.Cu) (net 7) (status 10))
 (segment (start 146.224 109.728) (end 146.224 109.808) (width 0.25) (layer F.Cu) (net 12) (status 30))
 (segment (start 146.224 109.808) (end 145.034 110.998) (width 0.25) (layer F.Cu) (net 12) (status 10))
 (segment (start 145.034 110.998) (end 145.034 113.03) (width 0.25) (layer F.Cu) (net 12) (status 20))
 (segment (start 139.5011 102.0036) (end 142.1356 102.0036) (width 0.25) (layer F.Cu) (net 13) (status 10))
 (segment (start 142.494 102.362) (end 142.494 113.03) (width 0.25) (layer F.Cu) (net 13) (status 20))
 (segment (start 142.1356 102.0036) (end 142.494 102.362) (width 0.25) (layer F.Cu) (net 13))
 (segment (start 139.954 109.554) (end 139.954 113.03) (width 0.25) (layer F.Cu) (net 10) (status 30))
 (segment (start 154.432 113.03) (end 153.162 111.76) (width 0.25) (layer F.Cu) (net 8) (status 10))
 (segment (start 154.0284 102.0036) (end 157.5011 102.0036) (width 0.25) (layer F.Cu) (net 8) (status 20))
 (segment (start 153.162 102.87) (end 154.0284 102.0036) (width 0.25) (layer F.Cu) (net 8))
 (segment (start 153.162 111.76) (end 153.162 102.87) (width 0.25) (layer F.Cu) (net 8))
 (segment (start 157.5011 100.5036) (end 153.0816 100.5036) (width 0.25) (layer F.Cu) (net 9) (status 10))
 (segment (start 151.892 101.6932) (end 151.892 113.03) (width 0.25) (layer F.Cu) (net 9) (status 20))
 (segment (start 153.0816 100.5036) (end 151.892 101.6932) (width 0.25) (layer F.Cu) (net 9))
 (segment (start 139.5011 93.0036) (end 144.3116 93.0036) (width 0.25) (layer F.Cu) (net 11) (status 10))
 (segment (start 146.224 94.916) (end 146.224 106.934) (width 0.25) (layer F.Cu) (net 11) (status 20))
 (segment (start 144.3116 93.0036) (end 146.224 94.916) (width 0.25) (layer F.Cu) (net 11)))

